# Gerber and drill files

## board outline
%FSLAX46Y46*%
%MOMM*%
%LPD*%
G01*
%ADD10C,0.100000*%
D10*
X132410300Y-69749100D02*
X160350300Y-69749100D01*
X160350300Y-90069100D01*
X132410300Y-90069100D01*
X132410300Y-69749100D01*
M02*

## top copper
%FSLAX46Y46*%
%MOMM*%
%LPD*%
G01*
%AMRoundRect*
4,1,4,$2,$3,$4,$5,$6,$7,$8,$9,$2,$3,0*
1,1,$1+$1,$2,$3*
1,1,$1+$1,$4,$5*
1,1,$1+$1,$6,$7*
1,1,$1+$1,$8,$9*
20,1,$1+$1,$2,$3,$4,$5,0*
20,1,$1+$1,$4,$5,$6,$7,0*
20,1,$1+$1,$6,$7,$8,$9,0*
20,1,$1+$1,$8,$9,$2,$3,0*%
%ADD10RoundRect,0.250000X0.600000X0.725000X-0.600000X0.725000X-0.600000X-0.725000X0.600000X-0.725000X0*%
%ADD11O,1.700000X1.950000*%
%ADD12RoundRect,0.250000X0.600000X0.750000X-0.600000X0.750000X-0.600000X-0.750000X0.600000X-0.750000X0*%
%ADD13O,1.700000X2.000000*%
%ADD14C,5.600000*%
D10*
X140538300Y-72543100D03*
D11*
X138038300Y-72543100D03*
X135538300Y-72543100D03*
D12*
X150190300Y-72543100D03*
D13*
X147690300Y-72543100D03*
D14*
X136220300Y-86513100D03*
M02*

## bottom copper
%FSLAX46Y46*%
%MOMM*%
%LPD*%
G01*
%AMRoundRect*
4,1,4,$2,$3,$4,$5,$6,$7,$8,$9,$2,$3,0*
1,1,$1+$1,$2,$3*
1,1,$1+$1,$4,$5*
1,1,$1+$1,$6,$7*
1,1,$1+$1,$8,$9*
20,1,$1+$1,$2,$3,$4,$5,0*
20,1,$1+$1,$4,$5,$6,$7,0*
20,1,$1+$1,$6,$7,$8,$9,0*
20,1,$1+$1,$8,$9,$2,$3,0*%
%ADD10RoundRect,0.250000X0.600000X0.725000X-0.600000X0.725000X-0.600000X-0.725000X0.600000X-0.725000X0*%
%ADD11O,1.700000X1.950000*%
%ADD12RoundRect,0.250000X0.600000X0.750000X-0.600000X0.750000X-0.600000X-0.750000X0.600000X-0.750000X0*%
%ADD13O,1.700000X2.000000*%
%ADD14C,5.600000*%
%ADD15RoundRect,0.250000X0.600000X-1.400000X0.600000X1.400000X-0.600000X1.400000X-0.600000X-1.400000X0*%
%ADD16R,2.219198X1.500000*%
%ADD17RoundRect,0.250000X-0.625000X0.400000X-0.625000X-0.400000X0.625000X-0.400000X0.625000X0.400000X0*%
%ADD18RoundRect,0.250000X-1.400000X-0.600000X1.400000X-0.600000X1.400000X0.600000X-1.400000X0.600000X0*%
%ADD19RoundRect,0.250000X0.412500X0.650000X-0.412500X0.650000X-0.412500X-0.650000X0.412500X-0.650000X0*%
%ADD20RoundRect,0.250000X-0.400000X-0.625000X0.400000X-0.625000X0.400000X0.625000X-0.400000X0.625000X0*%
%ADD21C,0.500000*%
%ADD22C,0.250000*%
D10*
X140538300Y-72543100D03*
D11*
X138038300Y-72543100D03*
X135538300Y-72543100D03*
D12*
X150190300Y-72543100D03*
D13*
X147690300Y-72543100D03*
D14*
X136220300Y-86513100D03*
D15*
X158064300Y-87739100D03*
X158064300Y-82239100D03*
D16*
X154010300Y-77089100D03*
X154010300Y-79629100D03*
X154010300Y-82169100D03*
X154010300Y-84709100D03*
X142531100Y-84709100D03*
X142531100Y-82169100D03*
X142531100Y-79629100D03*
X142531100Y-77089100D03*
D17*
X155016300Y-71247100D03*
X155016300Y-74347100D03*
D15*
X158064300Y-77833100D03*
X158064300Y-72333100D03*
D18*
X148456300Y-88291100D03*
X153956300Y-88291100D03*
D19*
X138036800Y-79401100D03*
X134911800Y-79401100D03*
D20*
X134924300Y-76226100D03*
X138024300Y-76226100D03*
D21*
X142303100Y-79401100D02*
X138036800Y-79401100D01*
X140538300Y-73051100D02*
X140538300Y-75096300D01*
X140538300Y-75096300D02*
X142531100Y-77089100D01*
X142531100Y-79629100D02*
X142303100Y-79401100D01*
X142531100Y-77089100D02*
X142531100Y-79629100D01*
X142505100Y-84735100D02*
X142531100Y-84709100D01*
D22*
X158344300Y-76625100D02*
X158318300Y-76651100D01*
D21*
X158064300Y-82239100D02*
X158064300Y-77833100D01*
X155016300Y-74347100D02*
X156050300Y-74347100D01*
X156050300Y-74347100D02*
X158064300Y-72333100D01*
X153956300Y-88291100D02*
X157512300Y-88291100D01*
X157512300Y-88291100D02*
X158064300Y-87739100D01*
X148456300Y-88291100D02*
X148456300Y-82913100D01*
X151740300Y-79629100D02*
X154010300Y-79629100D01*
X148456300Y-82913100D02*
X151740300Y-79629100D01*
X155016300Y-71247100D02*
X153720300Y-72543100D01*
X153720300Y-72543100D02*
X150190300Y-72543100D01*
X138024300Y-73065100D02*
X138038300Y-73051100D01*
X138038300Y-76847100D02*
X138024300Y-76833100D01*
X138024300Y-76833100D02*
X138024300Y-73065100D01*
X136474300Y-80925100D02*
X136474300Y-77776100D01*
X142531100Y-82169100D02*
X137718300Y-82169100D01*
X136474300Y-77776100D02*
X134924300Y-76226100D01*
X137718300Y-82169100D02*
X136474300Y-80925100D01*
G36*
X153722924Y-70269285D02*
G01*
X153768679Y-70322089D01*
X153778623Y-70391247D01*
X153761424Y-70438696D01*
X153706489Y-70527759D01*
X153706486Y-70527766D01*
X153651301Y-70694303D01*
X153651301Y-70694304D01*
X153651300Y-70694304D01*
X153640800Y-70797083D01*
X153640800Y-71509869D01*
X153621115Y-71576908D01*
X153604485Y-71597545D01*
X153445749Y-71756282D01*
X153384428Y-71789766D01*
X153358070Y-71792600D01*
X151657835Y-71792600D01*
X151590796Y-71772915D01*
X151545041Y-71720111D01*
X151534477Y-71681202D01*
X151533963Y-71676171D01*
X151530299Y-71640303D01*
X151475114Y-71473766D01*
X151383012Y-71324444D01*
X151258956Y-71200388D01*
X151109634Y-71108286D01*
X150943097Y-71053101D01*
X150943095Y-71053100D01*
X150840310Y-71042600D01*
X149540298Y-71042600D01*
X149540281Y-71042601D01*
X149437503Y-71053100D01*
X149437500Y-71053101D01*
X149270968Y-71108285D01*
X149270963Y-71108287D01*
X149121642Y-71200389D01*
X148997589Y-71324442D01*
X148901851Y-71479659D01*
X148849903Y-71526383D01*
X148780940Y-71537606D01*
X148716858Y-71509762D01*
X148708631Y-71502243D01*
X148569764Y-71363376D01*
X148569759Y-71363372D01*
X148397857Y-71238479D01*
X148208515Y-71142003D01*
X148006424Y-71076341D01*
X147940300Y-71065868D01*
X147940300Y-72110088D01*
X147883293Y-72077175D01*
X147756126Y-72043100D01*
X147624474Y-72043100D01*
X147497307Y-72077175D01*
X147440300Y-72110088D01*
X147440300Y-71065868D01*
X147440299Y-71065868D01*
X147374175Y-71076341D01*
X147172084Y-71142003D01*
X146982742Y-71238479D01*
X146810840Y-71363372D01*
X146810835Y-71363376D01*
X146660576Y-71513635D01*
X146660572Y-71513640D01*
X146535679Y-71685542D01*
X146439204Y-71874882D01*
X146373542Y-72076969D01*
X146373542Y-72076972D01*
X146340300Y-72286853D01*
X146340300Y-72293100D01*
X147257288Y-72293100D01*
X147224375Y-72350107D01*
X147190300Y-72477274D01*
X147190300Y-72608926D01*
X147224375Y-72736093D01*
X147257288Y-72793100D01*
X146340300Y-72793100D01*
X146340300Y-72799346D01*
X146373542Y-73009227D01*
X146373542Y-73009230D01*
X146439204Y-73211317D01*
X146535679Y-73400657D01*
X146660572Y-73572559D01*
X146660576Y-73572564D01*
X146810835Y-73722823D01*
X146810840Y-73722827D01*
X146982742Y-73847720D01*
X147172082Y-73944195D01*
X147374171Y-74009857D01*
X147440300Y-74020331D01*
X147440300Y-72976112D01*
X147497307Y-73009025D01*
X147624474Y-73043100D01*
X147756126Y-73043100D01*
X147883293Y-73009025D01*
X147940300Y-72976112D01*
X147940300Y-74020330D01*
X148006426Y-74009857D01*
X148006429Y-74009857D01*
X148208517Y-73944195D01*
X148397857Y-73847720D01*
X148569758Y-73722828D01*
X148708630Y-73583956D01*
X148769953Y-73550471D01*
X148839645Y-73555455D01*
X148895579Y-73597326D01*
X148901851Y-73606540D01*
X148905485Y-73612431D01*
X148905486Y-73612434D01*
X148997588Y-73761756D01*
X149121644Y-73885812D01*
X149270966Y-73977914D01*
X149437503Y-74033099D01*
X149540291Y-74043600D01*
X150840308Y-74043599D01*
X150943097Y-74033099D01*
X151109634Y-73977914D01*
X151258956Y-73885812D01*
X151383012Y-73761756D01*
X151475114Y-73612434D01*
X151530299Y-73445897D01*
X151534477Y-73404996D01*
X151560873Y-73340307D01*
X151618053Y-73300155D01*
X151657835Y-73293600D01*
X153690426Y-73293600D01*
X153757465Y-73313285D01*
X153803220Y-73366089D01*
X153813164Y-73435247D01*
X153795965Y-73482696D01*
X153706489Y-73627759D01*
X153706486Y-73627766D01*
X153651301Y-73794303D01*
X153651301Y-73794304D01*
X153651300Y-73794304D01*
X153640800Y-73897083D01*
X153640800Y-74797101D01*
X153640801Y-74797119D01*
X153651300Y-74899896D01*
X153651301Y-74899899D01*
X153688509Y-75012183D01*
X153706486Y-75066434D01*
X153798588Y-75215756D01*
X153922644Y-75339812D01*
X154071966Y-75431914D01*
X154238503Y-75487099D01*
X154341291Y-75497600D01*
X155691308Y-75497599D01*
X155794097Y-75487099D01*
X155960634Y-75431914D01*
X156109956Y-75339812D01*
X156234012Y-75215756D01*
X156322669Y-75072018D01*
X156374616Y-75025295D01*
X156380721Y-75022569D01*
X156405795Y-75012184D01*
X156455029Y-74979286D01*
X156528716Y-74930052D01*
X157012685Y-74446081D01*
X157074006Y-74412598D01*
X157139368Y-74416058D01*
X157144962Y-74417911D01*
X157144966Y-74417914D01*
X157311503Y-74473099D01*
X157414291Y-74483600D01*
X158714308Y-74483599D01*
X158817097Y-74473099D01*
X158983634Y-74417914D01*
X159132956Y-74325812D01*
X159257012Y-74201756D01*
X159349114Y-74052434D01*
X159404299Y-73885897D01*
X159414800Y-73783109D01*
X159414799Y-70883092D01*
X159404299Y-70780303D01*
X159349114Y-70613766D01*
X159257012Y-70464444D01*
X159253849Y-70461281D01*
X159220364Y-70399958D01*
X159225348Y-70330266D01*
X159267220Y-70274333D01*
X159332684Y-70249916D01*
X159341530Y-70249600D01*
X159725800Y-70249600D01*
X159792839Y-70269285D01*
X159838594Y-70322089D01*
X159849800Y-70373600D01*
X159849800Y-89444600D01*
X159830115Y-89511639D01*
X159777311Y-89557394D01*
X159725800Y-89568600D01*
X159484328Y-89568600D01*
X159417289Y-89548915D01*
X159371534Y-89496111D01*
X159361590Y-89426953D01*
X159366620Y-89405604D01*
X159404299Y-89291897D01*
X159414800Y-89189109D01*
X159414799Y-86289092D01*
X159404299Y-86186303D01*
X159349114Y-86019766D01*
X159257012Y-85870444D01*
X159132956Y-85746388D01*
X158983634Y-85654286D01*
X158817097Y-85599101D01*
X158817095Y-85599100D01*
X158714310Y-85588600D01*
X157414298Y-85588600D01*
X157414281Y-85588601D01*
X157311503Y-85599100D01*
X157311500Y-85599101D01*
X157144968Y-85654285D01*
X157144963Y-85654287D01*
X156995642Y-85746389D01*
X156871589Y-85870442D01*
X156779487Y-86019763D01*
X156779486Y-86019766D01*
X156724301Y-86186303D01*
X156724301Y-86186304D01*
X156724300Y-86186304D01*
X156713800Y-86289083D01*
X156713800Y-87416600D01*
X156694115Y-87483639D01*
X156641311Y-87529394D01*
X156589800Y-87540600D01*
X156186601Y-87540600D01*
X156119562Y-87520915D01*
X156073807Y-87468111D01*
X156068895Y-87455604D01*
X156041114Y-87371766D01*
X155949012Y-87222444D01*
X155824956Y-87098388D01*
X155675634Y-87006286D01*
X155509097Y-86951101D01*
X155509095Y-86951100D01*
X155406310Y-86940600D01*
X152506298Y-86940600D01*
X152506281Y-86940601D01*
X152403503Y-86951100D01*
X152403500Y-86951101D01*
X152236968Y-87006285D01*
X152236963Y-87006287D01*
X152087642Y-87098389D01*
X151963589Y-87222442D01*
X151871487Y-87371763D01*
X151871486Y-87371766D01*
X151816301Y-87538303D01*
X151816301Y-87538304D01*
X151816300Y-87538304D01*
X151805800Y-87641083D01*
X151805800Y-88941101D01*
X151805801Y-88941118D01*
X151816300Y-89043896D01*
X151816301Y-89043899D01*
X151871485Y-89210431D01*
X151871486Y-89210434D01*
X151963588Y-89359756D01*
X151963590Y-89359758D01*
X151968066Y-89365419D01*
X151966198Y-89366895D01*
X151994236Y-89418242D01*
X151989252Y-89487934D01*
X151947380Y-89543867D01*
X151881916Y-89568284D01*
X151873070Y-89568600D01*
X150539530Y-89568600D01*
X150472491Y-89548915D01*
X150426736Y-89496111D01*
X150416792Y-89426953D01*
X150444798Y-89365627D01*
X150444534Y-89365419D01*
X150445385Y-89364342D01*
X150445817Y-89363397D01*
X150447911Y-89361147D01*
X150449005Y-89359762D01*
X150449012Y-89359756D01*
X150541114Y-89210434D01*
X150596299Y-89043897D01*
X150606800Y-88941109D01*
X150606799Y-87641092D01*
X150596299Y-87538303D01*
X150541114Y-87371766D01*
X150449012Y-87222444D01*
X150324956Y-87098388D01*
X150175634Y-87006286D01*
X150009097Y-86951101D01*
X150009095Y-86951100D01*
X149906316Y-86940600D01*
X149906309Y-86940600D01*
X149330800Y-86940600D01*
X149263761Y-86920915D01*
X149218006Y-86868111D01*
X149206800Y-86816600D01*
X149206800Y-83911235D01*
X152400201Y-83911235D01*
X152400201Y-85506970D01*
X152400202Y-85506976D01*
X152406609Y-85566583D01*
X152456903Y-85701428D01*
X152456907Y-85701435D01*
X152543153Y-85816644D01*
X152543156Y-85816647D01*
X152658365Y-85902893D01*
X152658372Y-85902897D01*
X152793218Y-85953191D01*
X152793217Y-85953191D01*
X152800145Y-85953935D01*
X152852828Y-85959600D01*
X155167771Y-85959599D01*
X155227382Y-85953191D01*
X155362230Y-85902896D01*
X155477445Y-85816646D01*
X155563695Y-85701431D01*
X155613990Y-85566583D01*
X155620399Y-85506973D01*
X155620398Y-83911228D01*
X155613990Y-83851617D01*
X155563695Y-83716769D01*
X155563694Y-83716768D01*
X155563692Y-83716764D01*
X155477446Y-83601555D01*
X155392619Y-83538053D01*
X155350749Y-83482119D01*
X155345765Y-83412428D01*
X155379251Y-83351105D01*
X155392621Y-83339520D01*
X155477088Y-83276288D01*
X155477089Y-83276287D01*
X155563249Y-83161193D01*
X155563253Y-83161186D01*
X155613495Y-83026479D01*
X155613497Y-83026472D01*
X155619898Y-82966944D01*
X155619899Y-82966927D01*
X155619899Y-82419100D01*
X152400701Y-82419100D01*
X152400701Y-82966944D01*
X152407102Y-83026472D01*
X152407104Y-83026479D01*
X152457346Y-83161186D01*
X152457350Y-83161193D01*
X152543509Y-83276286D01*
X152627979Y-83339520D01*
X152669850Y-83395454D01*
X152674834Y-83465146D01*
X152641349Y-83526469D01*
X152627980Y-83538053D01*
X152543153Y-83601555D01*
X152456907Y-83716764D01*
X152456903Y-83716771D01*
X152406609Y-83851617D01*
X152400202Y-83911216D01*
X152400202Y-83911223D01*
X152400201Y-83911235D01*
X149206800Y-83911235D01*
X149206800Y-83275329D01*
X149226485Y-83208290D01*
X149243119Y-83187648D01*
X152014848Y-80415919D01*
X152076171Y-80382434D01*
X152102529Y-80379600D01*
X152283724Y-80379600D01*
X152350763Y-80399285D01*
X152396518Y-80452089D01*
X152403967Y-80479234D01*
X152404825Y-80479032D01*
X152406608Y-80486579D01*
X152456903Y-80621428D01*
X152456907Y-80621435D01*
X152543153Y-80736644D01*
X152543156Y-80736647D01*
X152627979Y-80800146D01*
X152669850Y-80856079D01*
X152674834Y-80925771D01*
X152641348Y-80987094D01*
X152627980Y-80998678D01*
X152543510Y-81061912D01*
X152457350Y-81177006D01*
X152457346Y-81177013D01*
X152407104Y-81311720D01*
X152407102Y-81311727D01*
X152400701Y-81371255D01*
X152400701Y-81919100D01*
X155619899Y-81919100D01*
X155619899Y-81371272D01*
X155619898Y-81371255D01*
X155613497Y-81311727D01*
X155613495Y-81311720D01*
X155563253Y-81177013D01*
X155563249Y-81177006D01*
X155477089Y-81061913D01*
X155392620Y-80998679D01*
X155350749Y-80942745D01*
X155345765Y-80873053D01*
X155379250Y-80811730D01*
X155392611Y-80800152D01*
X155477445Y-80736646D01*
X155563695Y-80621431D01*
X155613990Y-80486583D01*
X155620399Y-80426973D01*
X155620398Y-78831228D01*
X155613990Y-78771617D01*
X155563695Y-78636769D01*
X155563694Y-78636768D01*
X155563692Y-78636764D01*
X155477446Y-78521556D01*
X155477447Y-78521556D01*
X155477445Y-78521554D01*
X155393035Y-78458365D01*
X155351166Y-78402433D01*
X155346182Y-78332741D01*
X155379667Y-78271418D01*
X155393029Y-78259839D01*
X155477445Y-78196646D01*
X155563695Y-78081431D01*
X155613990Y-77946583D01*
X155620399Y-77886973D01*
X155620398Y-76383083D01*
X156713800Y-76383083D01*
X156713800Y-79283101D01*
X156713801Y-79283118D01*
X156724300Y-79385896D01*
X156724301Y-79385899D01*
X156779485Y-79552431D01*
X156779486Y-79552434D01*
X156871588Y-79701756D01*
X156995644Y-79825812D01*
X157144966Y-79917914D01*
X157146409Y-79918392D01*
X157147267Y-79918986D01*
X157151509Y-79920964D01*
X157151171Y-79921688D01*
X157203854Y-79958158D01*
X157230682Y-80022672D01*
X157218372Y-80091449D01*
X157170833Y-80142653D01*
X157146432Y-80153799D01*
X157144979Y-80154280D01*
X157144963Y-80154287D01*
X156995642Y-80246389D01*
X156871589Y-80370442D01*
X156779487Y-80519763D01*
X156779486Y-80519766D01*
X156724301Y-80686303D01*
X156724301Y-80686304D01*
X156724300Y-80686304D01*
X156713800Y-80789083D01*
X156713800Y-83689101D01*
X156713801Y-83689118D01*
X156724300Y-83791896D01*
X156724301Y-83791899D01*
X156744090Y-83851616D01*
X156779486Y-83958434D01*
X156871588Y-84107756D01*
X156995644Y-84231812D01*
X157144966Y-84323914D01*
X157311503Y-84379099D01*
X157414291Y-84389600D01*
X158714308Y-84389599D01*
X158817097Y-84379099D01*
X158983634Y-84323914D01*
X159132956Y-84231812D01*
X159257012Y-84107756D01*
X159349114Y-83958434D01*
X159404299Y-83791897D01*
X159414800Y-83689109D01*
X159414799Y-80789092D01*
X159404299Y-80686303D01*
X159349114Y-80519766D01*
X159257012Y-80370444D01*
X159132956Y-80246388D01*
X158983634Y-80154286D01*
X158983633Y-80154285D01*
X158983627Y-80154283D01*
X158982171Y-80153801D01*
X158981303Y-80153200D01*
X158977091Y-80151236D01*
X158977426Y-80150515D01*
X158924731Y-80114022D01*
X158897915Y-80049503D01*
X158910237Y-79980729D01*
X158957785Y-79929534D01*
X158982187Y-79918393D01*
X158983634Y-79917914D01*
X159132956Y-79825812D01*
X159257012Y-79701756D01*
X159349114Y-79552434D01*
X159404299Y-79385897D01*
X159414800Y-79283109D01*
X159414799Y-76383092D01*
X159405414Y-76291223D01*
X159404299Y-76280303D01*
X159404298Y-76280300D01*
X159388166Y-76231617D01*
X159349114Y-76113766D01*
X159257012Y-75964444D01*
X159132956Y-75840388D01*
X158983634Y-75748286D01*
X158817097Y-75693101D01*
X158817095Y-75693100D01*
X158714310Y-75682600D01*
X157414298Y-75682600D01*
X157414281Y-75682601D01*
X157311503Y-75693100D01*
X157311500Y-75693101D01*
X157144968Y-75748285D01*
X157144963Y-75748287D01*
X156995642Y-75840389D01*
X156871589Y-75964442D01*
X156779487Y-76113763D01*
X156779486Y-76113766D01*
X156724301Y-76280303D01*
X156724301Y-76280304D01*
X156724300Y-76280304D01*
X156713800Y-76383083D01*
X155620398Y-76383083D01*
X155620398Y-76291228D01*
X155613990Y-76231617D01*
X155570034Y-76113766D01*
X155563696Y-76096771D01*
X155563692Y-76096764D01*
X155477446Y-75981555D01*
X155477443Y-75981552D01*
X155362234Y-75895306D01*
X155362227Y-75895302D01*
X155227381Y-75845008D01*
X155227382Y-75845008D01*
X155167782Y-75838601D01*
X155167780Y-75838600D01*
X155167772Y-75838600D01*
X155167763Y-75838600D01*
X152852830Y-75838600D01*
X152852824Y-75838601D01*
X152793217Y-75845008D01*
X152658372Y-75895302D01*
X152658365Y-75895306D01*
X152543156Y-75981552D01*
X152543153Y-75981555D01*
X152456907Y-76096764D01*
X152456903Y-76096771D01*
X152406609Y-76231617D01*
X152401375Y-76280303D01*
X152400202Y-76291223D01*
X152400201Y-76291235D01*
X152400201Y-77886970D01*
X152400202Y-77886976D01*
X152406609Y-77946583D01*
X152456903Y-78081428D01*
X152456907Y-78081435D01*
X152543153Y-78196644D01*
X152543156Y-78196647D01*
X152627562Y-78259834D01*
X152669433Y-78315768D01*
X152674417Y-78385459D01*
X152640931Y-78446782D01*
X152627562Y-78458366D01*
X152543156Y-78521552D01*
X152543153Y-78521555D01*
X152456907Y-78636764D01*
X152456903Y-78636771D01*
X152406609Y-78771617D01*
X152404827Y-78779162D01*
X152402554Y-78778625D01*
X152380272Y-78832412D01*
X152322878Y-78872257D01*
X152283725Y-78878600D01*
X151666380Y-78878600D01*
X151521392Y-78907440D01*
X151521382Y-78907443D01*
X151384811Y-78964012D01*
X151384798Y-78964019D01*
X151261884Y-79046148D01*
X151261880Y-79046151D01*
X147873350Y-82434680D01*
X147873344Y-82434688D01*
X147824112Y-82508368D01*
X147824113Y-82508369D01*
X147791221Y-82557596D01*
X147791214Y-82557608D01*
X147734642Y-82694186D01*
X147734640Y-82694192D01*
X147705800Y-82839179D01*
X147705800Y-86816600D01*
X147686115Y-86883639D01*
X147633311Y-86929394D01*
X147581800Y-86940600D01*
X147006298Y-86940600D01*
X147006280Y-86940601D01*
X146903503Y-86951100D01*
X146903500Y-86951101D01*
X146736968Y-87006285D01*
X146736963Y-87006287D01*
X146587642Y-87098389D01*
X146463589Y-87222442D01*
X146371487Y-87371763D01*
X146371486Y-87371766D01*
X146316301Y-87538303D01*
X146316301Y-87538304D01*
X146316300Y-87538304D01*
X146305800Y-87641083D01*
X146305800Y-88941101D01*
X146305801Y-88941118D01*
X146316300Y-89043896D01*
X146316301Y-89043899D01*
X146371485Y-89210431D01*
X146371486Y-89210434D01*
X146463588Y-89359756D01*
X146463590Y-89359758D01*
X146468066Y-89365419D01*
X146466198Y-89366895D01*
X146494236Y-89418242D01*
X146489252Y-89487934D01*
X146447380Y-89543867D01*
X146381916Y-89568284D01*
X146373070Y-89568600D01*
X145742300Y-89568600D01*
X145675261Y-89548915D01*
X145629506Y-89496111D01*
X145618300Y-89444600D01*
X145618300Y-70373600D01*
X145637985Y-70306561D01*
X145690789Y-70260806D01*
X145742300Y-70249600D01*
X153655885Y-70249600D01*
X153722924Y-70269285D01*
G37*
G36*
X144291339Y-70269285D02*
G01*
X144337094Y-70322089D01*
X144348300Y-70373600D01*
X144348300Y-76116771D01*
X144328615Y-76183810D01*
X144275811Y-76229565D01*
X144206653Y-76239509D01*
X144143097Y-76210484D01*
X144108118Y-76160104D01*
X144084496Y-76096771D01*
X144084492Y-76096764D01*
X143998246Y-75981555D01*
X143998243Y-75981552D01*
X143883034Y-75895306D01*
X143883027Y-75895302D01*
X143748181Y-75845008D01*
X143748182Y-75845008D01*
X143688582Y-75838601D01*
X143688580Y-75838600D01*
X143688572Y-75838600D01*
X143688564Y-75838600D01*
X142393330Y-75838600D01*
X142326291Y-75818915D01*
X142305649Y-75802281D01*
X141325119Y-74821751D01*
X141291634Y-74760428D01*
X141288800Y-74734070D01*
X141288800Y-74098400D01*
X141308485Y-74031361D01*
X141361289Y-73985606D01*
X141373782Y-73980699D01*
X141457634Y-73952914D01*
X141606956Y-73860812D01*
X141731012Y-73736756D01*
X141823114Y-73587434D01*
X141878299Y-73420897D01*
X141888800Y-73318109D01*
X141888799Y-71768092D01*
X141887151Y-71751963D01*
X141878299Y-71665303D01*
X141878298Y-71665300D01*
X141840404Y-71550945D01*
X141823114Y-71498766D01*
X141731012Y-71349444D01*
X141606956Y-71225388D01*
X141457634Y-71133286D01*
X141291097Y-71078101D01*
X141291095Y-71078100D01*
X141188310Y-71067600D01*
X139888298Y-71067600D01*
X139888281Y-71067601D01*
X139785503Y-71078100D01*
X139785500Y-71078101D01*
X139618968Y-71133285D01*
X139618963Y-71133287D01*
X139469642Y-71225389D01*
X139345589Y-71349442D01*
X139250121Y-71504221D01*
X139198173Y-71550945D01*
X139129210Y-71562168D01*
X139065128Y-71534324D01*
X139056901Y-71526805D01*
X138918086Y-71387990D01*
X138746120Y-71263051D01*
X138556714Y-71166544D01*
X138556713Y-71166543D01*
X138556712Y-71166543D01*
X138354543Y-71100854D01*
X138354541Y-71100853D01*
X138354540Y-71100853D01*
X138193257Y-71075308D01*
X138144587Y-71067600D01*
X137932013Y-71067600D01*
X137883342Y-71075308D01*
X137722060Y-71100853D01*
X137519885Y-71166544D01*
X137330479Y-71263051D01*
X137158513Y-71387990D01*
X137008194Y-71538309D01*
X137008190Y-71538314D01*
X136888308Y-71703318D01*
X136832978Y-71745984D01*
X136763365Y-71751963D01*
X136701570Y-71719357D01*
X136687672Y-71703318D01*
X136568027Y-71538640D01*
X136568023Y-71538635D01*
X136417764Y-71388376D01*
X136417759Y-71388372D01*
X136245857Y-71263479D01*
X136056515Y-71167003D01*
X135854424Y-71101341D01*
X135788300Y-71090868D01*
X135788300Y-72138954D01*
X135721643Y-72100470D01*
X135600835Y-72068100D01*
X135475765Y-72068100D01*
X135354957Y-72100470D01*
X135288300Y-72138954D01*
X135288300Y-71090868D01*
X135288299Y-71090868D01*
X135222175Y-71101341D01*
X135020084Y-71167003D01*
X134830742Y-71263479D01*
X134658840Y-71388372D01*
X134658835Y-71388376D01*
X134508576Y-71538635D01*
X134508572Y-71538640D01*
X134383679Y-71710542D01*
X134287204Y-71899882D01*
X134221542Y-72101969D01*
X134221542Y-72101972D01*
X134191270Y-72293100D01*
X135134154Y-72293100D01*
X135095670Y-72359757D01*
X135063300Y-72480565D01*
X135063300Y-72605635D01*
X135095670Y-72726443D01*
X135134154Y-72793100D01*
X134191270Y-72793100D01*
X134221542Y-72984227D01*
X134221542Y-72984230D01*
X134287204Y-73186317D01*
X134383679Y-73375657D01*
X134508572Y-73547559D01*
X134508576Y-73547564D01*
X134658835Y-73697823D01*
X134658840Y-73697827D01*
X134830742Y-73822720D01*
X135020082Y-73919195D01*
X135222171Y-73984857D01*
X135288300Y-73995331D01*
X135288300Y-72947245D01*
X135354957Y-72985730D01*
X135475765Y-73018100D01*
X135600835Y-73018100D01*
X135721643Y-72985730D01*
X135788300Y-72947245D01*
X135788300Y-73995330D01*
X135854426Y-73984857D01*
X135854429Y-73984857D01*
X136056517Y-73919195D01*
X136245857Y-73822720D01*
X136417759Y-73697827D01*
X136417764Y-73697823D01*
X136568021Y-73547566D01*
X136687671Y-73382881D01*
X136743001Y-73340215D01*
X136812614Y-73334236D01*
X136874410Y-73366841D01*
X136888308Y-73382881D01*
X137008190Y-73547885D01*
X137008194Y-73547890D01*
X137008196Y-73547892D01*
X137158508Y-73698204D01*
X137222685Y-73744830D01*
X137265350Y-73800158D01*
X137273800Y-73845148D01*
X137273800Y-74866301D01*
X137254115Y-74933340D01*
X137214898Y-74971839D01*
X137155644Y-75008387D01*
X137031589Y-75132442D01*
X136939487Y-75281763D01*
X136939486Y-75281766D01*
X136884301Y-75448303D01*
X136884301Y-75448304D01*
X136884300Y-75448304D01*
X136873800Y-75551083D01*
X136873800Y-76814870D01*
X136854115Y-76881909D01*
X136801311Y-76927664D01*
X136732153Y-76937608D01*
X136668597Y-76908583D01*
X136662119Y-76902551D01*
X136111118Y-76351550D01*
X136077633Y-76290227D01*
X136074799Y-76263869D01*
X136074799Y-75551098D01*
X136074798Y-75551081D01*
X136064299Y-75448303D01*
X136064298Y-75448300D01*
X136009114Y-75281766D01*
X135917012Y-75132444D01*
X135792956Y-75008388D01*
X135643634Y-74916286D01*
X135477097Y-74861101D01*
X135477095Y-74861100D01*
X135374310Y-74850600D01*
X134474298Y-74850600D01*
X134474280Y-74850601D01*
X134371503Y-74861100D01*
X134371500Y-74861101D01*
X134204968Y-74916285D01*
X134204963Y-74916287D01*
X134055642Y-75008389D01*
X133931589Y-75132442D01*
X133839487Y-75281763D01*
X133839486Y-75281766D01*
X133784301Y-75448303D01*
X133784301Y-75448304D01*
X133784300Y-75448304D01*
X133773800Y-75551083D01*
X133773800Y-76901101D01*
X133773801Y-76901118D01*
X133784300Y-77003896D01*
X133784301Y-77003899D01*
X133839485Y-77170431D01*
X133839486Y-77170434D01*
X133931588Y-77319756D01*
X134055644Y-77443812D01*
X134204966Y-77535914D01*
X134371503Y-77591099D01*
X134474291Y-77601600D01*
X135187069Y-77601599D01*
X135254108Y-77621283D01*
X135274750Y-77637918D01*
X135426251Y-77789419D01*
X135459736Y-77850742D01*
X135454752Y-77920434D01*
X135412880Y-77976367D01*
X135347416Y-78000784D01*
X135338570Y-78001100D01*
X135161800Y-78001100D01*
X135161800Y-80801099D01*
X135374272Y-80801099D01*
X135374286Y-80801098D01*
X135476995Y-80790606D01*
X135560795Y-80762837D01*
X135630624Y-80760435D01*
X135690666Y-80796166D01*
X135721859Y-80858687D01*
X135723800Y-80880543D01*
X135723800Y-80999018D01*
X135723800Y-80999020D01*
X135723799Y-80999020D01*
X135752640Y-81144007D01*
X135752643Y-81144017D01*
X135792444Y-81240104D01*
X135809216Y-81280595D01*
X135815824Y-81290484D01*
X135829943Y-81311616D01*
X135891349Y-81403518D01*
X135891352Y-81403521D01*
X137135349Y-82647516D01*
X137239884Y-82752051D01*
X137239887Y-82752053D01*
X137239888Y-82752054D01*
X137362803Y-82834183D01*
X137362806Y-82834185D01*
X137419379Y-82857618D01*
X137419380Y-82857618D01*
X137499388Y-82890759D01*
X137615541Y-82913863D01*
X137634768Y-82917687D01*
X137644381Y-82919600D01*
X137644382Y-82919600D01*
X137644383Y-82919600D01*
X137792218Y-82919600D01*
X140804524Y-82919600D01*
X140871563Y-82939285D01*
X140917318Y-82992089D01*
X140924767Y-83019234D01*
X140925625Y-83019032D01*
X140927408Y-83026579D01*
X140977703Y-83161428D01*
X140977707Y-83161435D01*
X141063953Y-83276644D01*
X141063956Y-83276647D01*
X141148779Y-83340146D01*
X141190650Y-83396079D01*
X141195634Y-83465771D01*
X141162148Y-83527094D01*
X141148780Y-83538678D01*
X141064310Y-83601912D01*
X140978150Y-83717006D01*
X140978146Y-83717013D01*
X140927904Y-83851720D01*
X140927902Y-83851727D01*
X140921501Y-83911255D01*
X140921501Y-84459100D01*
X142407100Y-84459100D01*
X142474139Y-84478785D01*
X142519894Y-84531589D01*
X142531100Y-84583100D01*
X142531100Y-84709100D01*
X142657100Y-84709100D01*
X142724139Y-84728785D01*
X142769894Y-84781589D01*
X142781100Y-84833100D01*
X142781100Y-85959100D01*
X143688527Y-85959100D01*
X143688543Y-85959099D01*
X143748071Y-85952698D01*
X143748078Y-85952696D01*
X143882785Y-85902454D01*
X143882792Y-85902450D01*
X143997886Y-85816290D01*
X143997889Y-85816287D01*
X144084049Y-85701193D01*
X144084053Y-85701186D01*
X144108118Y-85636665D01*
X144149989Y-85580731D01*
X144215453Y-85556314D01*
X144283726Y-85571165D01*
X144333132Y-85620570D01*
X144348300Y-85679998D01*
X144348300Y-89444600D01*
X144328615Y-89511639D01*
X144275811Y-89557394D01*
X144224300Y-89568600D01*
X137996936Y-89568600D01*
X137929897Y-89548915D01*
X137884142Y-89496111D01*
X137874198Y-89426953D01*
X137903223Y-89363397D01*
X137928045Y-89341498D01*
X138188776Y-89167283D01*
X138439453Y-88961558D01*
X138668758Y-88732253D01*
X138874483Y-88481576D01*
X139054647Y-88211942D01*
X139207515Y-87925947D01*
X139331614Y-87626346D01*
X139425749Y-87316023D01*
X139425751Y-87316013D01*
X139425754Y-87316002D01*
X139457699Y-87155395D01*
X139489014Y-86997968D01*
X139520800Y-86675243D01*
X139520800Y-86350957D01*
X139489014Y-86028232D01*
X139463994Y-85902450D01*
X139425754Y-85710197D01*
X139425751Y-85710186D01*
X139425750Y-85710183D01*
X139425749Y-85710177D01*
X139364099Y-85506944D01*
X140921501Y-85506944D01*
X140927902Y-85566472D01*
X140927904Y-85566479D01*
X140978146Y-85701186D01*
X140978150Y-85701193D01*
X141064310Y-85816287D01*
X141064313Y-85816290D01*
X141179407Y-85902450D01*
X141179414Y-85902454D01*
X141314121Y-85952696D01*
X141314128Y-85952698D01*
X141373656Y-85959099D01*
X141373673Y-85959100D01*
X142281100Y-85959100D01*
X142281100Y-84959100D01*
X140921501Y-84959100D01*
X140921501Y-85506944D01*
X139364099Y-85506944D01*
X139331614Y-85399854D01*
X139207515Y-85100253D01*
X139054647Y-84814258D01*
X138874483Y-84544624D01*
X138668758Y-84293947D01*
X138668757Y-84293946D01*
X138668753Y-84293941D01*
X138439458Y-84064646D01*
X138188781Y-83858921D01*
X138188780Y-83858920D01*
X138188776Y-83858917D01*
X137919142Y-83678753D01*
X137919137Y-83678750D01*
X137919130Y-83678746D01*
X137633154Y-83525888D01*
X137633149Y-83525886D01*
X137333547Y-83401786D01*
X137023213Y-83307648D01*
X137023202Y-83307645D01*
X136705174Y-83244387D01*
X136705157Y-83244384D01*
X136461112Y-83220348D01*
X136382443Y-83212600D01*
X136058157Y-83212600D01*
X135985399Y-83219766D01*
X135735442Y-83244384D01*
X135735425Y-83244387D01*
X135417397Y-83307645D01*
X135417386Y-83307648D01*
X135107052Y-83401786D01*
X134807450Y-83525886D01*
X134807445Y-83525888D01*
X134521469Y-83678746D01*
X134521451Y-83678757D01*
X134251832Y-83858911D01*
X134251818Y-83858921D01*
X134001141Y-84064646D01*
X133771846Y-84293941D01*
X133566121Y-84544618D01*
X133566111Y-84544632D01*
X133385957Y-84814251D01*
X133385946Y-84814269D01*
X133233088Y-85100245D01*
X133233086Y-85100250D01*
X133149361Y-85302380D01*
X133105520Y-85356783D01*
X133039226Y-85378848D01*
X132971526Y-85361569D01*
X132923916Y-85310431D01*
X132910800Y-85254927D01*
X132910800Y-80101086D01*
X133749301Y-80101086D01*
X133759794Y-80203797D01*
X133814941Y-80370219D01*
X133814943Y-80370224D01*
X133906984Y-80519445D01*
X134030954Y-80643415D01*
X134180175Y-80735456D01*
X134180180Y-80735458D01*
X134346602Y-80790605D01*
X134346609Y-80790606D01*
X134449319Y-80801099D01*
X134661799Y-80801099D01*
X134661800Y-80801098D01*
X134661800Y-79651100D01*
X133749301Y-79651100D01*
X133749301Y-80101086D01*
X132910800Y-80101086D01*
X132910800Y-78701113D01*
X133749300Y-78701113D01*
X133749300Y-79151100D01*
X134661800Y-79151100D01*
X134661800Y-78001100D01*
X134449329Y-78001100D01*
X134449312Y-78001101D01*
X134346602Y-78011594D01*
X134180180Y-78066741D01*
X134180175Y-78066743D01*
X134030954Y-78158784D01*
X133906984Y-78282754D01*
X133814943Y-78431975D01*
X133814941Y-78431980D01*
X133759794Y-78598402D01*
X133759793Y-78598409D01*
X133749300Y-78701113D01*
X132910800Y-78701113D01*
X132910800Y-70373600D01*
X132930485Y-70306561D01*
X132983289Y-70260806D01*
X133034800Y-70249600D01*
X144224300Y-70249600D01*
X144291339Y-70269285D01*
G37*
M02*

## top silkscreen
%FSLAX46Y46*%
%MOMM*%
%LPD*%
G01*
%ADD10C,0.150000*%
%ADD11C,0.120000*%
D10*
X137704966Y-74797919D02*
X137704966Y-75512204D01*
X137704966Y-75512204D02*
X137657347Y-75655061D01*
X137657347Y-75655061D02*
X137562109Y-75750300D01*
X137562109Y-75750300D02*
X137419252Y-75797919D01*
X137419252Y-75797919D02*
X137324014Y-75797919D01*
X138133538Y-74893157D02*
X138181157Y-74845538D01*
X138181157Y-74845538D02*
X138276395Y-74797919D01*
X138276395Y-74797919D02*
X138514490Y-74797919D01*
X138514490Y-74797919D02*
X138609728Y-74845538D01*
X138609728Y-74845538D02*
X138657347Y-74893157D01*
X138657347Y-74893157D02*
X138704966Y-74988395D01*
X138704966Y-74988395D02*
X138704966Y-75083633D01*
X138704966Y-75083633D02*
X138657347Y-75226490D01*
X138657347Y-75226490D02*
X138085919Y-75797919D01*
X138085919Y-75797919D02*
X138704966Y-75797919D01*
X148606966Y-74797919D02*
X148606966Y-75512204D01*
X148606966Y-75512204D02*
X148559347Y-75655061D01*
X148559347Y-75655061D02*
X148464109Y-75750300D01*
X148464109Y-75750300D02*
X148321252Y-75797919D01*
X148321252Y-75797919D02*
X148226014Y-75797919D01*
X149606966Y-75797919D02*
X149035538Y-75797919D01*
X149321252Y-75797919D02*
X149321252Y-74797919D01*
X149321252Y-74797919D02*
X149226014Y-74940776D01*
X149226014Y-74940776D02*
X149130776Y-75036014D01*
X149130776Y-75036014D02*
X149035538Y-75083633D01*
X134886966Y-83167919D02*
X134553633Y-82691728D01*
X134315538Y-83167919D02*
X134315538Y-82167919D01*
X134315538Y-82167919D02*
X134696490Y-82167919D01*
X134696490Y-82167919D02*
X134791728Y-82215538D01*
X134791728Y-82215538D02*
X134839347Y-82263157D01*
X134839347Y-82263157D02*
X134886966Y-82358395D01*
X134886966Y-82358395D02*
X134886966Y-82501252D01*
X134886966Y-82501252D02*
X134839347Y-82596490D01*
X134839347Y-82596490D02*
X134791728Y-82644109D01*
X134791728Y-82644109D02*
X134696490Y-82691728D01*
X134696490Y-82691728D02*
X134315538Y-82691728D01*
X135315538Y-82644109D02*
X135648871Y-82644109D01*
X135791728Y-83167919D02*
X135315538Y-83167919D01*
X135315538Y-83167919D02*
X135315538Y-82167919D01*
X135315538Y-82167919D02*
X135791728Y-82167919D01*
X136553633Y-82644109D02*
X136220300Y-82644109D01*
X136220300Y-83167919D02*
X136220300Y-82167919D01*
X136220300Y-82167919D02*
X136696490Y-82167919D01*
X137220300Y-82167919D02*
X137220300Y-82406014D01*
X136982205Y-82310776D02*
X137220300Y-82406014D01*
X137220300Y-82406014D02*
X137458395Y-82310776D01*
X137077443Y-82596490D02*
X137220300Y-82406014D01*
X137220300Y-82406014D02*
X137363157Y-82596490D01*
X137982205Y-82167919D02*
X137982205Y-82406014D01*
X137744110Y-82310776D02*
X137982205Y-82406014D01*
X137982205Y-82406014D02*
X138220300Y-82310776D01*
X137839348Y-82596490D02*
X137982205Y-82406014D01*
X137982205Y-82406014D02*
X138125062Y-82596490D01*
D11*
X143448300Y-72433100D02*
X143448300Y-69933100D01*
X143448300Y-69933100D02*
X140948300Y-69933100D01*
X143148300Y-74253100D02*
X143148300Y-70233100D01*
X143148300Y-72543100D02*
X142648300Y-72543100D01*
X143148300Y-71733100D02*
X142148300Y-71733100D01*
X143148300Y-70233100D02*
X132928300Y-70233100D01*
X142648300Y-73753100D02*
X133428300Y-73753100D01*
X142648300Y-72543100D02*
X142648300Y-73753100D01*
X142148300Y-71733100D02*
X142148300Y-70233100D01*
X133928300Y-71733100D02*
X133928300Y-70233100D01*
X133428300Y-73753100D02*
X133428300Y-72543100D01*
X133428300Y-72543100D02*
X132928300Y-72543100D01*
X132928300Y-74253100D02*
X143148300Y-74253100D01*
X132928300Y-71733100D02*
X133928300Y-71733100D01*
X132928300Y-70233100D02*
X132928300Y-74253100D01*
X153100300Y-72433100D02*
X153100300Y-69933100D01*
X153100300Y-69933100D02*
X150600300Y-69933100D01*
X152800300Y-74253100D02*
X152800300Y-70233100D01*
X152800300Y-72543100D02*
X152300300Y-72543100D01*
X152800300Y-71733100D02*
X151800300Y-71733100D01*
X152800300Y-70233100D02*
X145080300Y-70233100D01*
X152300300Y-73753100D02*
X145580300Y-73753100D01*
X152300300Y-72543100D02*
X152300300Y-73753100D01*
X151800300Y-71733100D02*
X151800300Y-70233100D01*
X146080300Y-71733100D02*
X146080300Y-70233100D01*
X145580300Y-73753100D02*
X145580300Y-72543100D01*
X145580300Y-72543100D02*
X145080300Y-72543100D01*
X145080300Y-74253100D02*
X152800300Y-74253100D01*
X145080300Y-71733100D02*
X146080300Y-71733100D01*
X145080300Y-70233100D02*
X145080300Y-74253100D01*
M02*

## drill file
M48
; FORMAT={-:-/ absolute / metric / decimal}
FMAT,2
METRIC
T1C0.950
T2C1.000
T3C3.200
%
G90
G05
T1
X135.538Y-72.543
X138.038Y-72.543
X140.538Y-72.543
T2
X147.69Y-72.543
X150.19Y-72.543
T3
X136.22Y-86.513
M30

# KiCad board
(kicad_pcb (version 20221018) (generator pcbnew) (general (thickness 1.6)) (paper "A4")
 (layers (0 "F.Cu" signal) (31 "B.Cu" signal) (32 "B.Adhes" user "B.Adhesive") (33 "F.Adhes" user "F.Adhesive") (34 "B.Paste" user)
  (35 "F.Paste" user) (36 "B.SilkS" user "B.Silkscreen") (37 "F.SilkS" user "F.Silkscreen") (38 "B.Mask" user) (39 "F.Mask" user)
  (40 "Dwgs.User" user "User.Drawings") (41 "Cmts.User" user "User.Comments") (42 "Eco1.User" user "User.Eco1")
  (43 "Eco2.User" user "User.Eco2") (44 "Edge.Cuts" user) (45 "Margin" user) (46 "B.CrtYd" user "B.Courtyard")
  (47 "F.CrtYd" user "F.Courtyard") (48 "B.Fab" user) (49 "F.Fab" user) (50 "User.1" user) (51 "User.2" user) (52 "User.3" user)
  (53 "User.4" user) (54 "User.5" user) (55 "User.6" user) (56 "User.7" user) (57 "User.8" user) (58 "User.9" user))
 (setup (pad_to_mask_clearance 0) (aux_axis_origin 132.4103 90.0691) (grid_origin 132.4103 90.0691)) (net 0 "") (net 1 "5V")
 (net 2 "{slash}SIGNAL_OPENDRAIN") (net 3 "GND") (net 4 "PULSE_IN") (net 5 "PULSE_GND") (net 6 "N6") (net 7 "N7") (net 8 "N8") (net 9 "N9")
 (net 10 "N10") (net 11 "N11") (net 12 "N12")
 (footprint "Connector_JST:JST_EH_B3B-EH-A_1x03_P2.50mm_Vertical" (layer "F.Cu") (at 140.5383 72.5431 180)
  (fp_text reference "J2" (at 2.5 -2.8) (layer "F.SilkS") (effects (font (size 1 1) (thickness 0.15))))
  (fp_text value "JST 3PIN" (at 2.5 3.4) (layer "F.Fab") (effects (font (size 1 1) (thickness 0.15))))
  (fp_line (start -2.91 0.11) (end -2.91 2.61) (stroke (width 0.12) (type solid)) (layer "F.SilkS"))
  (fp_line (start -2.91 2.61) (end -0.41 2.61) (stroke (width 0.12) (type solid)) (layer "F.SilkS"))
  (fp_line (start -2.61 -1.71) (end -2.61 2.31) (stroke (width 0.12) (type solid)) (layer "F.SilkS"))
  (fp_line (start -2.61 0) (end -2.11 0) (stroke (width 0.12) (type solid)) (layer "F.SilkS"))
  (fp_line (start -2.61 0.81) (end -1.61 0.81) (stroke (width 0.12) (type solid)) (layer "F.SilkS"))
  (fp_line (start -2.61 2.31) (end 7.61 2.31) (stroke (width 0.12) (type solid)) (layer "F.SilkS"))
  (fp_line (start -2.11 -1.21) (end 7.11 -1.21) (stroke (width 0.12) (type solid)) (layer "F.SilkS"))
  (fp_line (start -2.11 0) (end -2.11 -1.21) (stroke (width 0.12) (type solid)) (layer "F.SilkS"))
  (fp_line (start -1.61 0.81) (end -1.61 2.31) (stroke (width 0.12) (type solid)) (layer "F.SilkS"))
  (fp_line (start 6.61 0.81) (end 6.61 2.31) (stroke (width 0.12) (type solid)) (layer "F.SilkS"))
  (fp_line (start 7.11 -1.21) (end 7.11 0) (stroke (width 0.12) (type solid)) (layer "F.SilkS"))
  (fp_line (start 7.11 0) (end 7.61 0) (stroke (width 0.12) (type solid)) (layer "F.SilkS"))
  (fp_line (start 7.61 -1.71) (end -2.61 -1.71) (stroke (width 0.12) (type solid)) (layer "F.SilkS"))
  (fp_line (start 7.61 0.81) (end 6.61 0.81) (stroke (width 0.12) (type solid)) (layer "F.SilkS"))
  (fp_line (start 7.61 2.31) (end 7.61 -1.71) (stroke (width 0.12) (type solid)) (layer "F.SilkS"))
  (pad "1" thru_hole roundrect (at 0 0 180) (size 1.7 1.95) (drill 0.95) (layers "*.Cu" "*.Mask") (roundrect_rratio 0.1470588235)
   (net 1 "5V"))
  (pad "2" thru_hole oval (at 2.5 0 180) (size 1.7 1.95) (drill 0.95) (layers "*.Cu" "*.Mask") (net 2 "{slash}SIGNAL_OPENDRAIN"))
  (pad "3" thru_hole oval (at 5 0 180) (size 1.7 1.95) (drill 0.95) (layers "*.Cu" "*.Mask") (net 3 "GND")))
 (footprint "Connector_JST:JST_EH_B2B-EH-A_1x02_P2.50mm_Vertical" (layer "F.Cu") (at 150.1903 72.5431 180)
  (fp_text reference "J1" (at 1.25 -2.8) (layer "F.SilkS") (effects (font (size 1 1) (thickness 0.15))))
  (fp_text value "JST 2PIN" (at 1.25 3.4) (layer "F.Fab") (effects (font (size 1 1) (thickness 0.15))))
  (fp_line (start -2.91 0.11) (end -2.91 2.61) (stroke (width 0.12) (type solid)) (layer "F.SilkS"))
  (fp_line (start -2.91 2.61) (end -0.41 2.61) (stroke (width 0.12) (type solid)) (layer "F.SilkS"))
  (fp_line (start -2.61 -1.71) (end -2.61 2.31) (stroke (width 0.12) (type solid)) (layer "F.SilkS"))
  (fp_line (start -2.61 0) (end -2.11 0) (stroke (width 0.12) (type solid)) (layer "F.SilkS"))
  (fp_line (start -2.61 0.81) (end -1.61 0.81) (stroke (width 0.12) (type solid)) (layer "F.SilkS"))
  (fp_line (start -2.61 2.31) (end 5.11 2.31) (stroke (width 0.12) (type solid)) (layer "F.SilkS"))
  (fp_line (start -2.11 -1.21) (end 4.61 -1.21) (stroke (width 0.12) (type solid)) (layer "F.SilkS"))
  (fp_line (start -2.11 0) (end -2.11 -1.21) (stroke (width 0.12) (type solid)) (layer "F.SilkS"))
  (fp_line (start -1.61 0.81) (end -1.61 2.31) (stroke (width 0.12) (type solid)) (layer "F.SilkS"))
  (fp_line (start 4.11 0.81) (end 4.11 2.31) (stroke (width 0.12) (type solid)) (layer "F.SilkS"))
  (fp_line (start 4.61 -1.21) (end 4.61 0) (stroke (width 0.12) (type solid)) (layer "F.SilkS"))
  (fp_line (start 4.61 0) (end 5.11 0) (stroke (width 0.12) (type solid)) (layer "F.SilkS"))
  (fp_line (start 5.11 -1.71) (end -2.61 -1.71) (stroke (width 0.12) (type solid)) (layer "F.SilkS"))
  (fp_line (start 5.11 0.81) (end 4.11 0.81) (stroke (width 0.12) (type solid)) (layer "F.SilkS"))
  (fp_line (start 5.11 2.31) (end 5.11 -1.71) (stroke (width 0.12) (type solid)) (layer "F.SilkS"))
  (pad "1" thru_hole roundrect (at 0 0 180) (size 1.7 2) (drill 1) (layers "*.Cu" "*.Mask") (roundrect_rratio 0.1470588235)
   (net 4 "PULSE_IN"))
  (pad "2" thru_hole oval (at 2.5 0 180) (size 1.7 2) (drill 1) (layers "*.Cu" "*.Mask") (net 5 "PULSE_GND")))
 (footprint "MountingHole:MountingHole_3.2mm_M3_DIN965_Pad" (layer "F.Cu") (at 136.2203 86.5131)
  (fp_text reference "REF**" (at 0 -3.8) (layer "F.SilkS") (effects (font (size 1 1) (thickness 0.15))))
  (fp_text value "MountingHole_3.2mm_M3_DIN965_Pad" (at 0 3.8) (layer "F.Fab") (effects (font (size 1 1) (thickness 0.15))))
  (pad "1" thru_hole circle (at 0 0) (size 5.6 5.6) (drill 3.2) (layers "*.Cu" "*.Mask")))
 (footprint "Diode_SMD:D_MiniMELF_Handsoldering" (layer "B.Cu") (at 158.0643 84.9891 90)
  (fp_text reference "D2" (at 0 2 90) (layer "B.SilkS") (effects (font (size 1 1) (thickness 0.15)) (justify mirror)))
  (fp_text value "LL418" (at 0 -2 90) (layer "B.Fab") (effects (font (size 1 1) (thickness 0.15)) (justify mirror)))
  (pad "1" smd roundrect (at -2.75 0 90) (size 3.3 1.7) (layers "B.Cu" "B.Paste" "B.Mask") (roundrect_rratio 0.1470588235) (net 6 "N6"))
  (pad "2" smd roundrect (at 2.75 0 90) (size 3.3 1.7) (layers "B.Cu" "B.Paste" "B.Mask") (roundrect_rratio 0.1470588235) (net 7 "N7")))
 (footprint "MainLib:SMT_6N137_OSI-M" (layer "B.Cu") (at 148.2707 80.8991 180)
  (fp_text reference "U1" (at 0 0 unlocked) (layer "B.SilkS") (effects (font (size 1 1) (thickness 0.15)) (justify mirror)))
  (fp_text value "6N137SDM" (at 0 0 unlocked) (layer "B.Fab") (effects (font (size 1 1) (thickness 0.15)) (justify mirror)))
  (pad "1" smd rect (at -5.7396 3.81 180) (size 2.219198 1.5) (layers "B.Cu" "B.Paste" "B.Mask") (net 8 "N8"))
  (pad "2" smd rect (at -5.7396 1.27 180) (size 2.219198 1.5) (layers "B.Cu" "B.Paste" "B.Mask") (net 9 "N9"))
  (pad "3" smd rect (at -5.7396 -1.27 180) (size 2.219198 1.5) (layers "B.Cu" "B.Paste" "B.Mask") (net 5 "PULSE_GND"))
  (pad "4" smd rect (at -5.7396 -3.81 180) (size 2.219198 1.5) (layers "B.Cu" "B.Paste" "B.Mask") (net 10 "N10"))
  (pad "5" smd rect (at 5.7396 -3.81 180) (size 2.219198 1.5) (layers "B.Cu" "B.Paste" "B.Mask") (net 3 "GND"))
  (pad "6" smd rect (at 5.7396 -1.27 180) (size 2.219198 1.5) (layers "B.Cu" "B.Paste" "B.Mask") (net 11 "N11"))
  (pad "7" smd rect (at 5.7396 1.27 180) (size 2.219198 1.5) (layers "B.Cu" "B.Paste" "B.Mask") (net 1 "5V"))
  (pad "8" smd rect (at 5.7396 3.81 180) (size 2.219198 1.5) (layers "B.Cu" "B.Paste" "B.Mask") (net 1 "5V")))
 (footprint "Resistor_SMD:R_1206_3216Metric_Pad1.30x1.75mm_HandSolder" (layer "B.Cu") (at 155.0163 72.7971 -90)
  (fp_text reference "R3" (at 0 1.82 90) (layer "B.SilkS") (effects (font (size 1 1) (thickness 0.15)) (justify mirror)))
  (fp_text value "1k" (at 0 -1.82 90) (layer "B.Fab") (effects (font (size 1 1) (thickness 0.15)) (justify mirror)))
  (pad "1" smd roundrect (at -1.55 0 270) (size 1.3 1.75) (layers "B.Cu" "B.Paste" "B.Mask") (roundrect_rratio 0.1923076923)
   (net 4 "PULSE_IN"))
  (pad "2" smd roundrect (at 1.55 0 270) (size 1.3 1.75) (layers "B.Cu" "B.Paste" "B.Mask") (roundrect_rratio 0.1923076923) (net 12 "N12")))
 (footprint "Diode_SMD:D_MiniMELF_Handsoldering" (layer "B.Cu") (at 158.0643 75.0831 90)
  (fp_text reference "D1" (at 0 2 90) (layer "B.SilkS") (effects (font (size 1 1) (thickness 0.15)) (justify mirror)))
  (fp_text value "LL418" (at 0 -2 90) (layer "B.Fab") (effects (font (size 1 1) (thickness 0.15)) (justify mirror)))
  (pad "1" smd roundrect (at -2.75 0 90) (size 3.3 1.7) (layers "B.Cu" "B.Paste" "B.Mask") (roundrect_rratio 0.1470588235) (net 7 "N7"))
  (pad "2" smd roundrect (at 2.75 0 90) (size 3.3 1.7) (layers "B.Cu" "B.Paste" "B.Mask") (roundrect_rratio 0.1470588235) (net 12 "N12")))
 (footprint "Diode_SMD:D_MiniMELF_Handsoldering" (layer "B.Cu") (at 151.2063 88.2911)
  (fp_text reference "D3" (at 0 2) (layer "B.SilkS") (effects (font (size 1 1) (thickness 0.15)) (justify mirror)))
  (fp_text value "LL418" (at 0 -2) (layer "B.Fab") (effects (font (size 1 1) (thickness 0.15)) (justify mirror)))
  (pad "1" smd roundrect (at -2.75 0) (size 3.3 1.7) (layers "B.Cu" "B.Paste" "B.Mask") (roundrect_rratio 0.1470588235) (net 9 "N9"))
  (pad "2" smd roundrect (at 2.75 0) (size 3.3 1.7) (layers "B.Cu" "B.Paste" "B.Mask") (roundrect_rratio 0.1470588235) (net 6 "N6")))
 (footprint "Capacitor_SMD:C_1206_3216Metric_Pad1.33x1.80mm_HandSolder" (layer "B.Cu") (at 136.4743 79.4011 180)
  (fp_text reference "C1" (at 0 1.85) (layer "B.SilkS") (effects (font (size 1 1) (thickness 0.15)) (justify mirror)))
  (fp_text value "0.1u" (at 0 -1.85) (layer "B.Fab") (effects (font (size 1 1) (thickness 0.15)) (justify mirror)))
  (pad "1" smd roundrect (at -1.5625 0 180) (size 1.325 1.8) (layers "B.Cu" "B.Paste" "B.Mask") (roundrect_rratio 0.1886792453) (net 1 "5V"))
  (pad "2" smd roundrect (at 1.5625 0 180) (size 1.325 1.8) (layers "B.Cu" "B.Paste" "B.Mask") (roundrect_rratio 0.1886792453) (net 3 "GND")))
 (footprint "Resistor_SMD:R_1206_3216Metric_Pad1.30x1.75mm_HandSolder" (layer "B.Cu") (at 136.4743 76.2261)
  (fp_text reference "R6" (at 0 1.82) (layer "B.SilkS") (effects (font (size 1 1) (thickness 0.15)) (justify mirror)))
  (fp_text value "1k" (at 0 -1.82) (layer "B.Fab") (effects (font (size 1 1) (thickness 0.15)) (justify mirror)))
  (pad "1" smd roundrect (at -1.55 0) (size 1.3 1.75) (layers "B.Cu" "B.Paste" "B.Mask") (roundrect_rratio 0.1923076923) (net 11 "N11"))
  (pad "2" smd roundrect (at 1.55 0) (size 1.3 1.75) (layers "B.Cu" "B.Paste" "B.Mask") (roundrect_rratio 0.1923076923)
   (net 2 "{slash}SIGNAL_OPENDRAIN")))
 (gr_rect (start 132.4103 69.7491) (end 160.3503 90.0691) (stroke (width 0.1) (type default)) (fill none) (layer "Edge.Cuts"))
 (segment (start 142.3031 79.4011) (end 138.0368 79.4011) (width 0.5) (layer "B.Cu") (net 1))
 (segment (start 140.5383 73.0511) (end 140.5383 75.0963) (width 0.5) (layer "B.Cu") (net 1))
 (segment (start 140.5383 75.0963) (end 142.5311 77.0891) (width 0.5) (layer "B.Cu") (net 1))
 (segment (start 142.5311 79.6291) (end 142.3031 79.4011) (width 0.5) (layer "B.Cu") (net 1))
 (segment (start 142.5311 77.0891) (end 142.5311 79.6291) (width 0.5) (layer "B.Cu") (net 1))
 (segment (start 142.5051 84.7351) (end 142.5311 84.7091) (width 0.5) (layer "B.Cu") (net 3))
 (segment (start 158.3443 76.6251) (end 158.3183 76.6511) (width 0.25) (layer "B.Cu") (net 7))
 (segment (start 158.0643 82.2391) (end 158.0643 77.8331) (width 0.5) (layer "B.Cu") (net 7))
 (segment (start 155.0163 74.3471) (end 156.0503 74.3471) (width 0.5) (layer "B.Cu") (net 12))
 (segment (start 156.0503 74.3471) (end 158.0643 72.3331) (width 0.5) (layer "B.Cu") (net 12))
 (segment (start 153.9563 88.2911) (end 157.5123 88.2911) (width 0.5) (layer "B.Cu") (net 6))
 (segment (start 157.5123 88.2911) (end 158.0643 87.7391) (width 0.5) (layer "B.Cu") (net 6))
 (segment (start 148.4563 88.2911) (end 148.4563 82.9131) (width 0.5) (layer "B.Cu") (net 9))
 (segment (start 151.7403 79.6291) (end 154.0103 79.6291) (width 0.5) (layer "B.Cu") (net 9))
 (segment (start 148.4563 82.9131) (end 151.7403 79.6291) (width 0.5) (layer "B.Cu") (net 9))
 (segment (start 155.0163 71.2471) (end 153.7203 72.5431) (width 0.5) (layer "B.Cu") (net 4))
 (segment (start 153.7203 72.5431) (end 150.1903 72.5431) (width 0.5) (layer "B.Cu") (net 4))
 (segment (start 138.0243 73.0651) (end 138.0383 73.0511) (width 0.5) (layer "B.Cu") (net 2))
 (segment (start 138.0383 76.8471) (end 138.0243 76.8331) (width 0.5) (layer "B.Cu") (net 2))
 (segment (start 138.0243 76.8331) (end 138.0243 73.0651) (width 0.5) (layer "B.Cu") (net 2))
 (segment (start 136.4743 80.9251) (end 136.4743 77.7761) (width 0.5) (layer "B.Cu") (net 11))
 (segment (start 142.5311 82.1691) (end 137.7183 82.1691) (width 0.5) (layer "B.Cu") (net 11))
 (segment (start 136.4743 77.7761) (end 134.9243 76.2261) (width 0.5) (layer "B.Cu") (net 11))
 (segment (start 137.7183 82.1691) (end 136.4743 80.9251) (width 0.5) (layer "B.Cu") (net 11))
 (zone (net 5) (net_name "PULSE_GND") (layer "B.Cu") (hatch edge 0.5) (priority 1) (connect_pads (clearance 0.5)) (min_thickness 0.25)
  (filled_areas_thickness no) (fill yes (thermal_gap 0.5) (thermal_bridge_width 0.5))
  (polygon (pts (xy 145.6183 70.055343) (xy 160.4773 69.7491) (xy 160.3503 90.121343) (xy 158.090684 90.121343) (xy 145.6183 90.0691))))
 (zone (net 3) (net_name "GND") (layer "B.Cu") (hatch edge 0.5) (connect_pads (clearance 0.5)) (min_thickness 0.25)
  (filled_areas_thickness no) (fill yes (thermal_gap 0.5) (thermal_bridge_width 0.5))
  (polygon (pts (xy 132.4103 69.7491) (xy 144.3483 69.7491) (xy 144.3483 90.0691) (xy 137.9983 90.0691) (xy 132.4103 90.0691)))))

